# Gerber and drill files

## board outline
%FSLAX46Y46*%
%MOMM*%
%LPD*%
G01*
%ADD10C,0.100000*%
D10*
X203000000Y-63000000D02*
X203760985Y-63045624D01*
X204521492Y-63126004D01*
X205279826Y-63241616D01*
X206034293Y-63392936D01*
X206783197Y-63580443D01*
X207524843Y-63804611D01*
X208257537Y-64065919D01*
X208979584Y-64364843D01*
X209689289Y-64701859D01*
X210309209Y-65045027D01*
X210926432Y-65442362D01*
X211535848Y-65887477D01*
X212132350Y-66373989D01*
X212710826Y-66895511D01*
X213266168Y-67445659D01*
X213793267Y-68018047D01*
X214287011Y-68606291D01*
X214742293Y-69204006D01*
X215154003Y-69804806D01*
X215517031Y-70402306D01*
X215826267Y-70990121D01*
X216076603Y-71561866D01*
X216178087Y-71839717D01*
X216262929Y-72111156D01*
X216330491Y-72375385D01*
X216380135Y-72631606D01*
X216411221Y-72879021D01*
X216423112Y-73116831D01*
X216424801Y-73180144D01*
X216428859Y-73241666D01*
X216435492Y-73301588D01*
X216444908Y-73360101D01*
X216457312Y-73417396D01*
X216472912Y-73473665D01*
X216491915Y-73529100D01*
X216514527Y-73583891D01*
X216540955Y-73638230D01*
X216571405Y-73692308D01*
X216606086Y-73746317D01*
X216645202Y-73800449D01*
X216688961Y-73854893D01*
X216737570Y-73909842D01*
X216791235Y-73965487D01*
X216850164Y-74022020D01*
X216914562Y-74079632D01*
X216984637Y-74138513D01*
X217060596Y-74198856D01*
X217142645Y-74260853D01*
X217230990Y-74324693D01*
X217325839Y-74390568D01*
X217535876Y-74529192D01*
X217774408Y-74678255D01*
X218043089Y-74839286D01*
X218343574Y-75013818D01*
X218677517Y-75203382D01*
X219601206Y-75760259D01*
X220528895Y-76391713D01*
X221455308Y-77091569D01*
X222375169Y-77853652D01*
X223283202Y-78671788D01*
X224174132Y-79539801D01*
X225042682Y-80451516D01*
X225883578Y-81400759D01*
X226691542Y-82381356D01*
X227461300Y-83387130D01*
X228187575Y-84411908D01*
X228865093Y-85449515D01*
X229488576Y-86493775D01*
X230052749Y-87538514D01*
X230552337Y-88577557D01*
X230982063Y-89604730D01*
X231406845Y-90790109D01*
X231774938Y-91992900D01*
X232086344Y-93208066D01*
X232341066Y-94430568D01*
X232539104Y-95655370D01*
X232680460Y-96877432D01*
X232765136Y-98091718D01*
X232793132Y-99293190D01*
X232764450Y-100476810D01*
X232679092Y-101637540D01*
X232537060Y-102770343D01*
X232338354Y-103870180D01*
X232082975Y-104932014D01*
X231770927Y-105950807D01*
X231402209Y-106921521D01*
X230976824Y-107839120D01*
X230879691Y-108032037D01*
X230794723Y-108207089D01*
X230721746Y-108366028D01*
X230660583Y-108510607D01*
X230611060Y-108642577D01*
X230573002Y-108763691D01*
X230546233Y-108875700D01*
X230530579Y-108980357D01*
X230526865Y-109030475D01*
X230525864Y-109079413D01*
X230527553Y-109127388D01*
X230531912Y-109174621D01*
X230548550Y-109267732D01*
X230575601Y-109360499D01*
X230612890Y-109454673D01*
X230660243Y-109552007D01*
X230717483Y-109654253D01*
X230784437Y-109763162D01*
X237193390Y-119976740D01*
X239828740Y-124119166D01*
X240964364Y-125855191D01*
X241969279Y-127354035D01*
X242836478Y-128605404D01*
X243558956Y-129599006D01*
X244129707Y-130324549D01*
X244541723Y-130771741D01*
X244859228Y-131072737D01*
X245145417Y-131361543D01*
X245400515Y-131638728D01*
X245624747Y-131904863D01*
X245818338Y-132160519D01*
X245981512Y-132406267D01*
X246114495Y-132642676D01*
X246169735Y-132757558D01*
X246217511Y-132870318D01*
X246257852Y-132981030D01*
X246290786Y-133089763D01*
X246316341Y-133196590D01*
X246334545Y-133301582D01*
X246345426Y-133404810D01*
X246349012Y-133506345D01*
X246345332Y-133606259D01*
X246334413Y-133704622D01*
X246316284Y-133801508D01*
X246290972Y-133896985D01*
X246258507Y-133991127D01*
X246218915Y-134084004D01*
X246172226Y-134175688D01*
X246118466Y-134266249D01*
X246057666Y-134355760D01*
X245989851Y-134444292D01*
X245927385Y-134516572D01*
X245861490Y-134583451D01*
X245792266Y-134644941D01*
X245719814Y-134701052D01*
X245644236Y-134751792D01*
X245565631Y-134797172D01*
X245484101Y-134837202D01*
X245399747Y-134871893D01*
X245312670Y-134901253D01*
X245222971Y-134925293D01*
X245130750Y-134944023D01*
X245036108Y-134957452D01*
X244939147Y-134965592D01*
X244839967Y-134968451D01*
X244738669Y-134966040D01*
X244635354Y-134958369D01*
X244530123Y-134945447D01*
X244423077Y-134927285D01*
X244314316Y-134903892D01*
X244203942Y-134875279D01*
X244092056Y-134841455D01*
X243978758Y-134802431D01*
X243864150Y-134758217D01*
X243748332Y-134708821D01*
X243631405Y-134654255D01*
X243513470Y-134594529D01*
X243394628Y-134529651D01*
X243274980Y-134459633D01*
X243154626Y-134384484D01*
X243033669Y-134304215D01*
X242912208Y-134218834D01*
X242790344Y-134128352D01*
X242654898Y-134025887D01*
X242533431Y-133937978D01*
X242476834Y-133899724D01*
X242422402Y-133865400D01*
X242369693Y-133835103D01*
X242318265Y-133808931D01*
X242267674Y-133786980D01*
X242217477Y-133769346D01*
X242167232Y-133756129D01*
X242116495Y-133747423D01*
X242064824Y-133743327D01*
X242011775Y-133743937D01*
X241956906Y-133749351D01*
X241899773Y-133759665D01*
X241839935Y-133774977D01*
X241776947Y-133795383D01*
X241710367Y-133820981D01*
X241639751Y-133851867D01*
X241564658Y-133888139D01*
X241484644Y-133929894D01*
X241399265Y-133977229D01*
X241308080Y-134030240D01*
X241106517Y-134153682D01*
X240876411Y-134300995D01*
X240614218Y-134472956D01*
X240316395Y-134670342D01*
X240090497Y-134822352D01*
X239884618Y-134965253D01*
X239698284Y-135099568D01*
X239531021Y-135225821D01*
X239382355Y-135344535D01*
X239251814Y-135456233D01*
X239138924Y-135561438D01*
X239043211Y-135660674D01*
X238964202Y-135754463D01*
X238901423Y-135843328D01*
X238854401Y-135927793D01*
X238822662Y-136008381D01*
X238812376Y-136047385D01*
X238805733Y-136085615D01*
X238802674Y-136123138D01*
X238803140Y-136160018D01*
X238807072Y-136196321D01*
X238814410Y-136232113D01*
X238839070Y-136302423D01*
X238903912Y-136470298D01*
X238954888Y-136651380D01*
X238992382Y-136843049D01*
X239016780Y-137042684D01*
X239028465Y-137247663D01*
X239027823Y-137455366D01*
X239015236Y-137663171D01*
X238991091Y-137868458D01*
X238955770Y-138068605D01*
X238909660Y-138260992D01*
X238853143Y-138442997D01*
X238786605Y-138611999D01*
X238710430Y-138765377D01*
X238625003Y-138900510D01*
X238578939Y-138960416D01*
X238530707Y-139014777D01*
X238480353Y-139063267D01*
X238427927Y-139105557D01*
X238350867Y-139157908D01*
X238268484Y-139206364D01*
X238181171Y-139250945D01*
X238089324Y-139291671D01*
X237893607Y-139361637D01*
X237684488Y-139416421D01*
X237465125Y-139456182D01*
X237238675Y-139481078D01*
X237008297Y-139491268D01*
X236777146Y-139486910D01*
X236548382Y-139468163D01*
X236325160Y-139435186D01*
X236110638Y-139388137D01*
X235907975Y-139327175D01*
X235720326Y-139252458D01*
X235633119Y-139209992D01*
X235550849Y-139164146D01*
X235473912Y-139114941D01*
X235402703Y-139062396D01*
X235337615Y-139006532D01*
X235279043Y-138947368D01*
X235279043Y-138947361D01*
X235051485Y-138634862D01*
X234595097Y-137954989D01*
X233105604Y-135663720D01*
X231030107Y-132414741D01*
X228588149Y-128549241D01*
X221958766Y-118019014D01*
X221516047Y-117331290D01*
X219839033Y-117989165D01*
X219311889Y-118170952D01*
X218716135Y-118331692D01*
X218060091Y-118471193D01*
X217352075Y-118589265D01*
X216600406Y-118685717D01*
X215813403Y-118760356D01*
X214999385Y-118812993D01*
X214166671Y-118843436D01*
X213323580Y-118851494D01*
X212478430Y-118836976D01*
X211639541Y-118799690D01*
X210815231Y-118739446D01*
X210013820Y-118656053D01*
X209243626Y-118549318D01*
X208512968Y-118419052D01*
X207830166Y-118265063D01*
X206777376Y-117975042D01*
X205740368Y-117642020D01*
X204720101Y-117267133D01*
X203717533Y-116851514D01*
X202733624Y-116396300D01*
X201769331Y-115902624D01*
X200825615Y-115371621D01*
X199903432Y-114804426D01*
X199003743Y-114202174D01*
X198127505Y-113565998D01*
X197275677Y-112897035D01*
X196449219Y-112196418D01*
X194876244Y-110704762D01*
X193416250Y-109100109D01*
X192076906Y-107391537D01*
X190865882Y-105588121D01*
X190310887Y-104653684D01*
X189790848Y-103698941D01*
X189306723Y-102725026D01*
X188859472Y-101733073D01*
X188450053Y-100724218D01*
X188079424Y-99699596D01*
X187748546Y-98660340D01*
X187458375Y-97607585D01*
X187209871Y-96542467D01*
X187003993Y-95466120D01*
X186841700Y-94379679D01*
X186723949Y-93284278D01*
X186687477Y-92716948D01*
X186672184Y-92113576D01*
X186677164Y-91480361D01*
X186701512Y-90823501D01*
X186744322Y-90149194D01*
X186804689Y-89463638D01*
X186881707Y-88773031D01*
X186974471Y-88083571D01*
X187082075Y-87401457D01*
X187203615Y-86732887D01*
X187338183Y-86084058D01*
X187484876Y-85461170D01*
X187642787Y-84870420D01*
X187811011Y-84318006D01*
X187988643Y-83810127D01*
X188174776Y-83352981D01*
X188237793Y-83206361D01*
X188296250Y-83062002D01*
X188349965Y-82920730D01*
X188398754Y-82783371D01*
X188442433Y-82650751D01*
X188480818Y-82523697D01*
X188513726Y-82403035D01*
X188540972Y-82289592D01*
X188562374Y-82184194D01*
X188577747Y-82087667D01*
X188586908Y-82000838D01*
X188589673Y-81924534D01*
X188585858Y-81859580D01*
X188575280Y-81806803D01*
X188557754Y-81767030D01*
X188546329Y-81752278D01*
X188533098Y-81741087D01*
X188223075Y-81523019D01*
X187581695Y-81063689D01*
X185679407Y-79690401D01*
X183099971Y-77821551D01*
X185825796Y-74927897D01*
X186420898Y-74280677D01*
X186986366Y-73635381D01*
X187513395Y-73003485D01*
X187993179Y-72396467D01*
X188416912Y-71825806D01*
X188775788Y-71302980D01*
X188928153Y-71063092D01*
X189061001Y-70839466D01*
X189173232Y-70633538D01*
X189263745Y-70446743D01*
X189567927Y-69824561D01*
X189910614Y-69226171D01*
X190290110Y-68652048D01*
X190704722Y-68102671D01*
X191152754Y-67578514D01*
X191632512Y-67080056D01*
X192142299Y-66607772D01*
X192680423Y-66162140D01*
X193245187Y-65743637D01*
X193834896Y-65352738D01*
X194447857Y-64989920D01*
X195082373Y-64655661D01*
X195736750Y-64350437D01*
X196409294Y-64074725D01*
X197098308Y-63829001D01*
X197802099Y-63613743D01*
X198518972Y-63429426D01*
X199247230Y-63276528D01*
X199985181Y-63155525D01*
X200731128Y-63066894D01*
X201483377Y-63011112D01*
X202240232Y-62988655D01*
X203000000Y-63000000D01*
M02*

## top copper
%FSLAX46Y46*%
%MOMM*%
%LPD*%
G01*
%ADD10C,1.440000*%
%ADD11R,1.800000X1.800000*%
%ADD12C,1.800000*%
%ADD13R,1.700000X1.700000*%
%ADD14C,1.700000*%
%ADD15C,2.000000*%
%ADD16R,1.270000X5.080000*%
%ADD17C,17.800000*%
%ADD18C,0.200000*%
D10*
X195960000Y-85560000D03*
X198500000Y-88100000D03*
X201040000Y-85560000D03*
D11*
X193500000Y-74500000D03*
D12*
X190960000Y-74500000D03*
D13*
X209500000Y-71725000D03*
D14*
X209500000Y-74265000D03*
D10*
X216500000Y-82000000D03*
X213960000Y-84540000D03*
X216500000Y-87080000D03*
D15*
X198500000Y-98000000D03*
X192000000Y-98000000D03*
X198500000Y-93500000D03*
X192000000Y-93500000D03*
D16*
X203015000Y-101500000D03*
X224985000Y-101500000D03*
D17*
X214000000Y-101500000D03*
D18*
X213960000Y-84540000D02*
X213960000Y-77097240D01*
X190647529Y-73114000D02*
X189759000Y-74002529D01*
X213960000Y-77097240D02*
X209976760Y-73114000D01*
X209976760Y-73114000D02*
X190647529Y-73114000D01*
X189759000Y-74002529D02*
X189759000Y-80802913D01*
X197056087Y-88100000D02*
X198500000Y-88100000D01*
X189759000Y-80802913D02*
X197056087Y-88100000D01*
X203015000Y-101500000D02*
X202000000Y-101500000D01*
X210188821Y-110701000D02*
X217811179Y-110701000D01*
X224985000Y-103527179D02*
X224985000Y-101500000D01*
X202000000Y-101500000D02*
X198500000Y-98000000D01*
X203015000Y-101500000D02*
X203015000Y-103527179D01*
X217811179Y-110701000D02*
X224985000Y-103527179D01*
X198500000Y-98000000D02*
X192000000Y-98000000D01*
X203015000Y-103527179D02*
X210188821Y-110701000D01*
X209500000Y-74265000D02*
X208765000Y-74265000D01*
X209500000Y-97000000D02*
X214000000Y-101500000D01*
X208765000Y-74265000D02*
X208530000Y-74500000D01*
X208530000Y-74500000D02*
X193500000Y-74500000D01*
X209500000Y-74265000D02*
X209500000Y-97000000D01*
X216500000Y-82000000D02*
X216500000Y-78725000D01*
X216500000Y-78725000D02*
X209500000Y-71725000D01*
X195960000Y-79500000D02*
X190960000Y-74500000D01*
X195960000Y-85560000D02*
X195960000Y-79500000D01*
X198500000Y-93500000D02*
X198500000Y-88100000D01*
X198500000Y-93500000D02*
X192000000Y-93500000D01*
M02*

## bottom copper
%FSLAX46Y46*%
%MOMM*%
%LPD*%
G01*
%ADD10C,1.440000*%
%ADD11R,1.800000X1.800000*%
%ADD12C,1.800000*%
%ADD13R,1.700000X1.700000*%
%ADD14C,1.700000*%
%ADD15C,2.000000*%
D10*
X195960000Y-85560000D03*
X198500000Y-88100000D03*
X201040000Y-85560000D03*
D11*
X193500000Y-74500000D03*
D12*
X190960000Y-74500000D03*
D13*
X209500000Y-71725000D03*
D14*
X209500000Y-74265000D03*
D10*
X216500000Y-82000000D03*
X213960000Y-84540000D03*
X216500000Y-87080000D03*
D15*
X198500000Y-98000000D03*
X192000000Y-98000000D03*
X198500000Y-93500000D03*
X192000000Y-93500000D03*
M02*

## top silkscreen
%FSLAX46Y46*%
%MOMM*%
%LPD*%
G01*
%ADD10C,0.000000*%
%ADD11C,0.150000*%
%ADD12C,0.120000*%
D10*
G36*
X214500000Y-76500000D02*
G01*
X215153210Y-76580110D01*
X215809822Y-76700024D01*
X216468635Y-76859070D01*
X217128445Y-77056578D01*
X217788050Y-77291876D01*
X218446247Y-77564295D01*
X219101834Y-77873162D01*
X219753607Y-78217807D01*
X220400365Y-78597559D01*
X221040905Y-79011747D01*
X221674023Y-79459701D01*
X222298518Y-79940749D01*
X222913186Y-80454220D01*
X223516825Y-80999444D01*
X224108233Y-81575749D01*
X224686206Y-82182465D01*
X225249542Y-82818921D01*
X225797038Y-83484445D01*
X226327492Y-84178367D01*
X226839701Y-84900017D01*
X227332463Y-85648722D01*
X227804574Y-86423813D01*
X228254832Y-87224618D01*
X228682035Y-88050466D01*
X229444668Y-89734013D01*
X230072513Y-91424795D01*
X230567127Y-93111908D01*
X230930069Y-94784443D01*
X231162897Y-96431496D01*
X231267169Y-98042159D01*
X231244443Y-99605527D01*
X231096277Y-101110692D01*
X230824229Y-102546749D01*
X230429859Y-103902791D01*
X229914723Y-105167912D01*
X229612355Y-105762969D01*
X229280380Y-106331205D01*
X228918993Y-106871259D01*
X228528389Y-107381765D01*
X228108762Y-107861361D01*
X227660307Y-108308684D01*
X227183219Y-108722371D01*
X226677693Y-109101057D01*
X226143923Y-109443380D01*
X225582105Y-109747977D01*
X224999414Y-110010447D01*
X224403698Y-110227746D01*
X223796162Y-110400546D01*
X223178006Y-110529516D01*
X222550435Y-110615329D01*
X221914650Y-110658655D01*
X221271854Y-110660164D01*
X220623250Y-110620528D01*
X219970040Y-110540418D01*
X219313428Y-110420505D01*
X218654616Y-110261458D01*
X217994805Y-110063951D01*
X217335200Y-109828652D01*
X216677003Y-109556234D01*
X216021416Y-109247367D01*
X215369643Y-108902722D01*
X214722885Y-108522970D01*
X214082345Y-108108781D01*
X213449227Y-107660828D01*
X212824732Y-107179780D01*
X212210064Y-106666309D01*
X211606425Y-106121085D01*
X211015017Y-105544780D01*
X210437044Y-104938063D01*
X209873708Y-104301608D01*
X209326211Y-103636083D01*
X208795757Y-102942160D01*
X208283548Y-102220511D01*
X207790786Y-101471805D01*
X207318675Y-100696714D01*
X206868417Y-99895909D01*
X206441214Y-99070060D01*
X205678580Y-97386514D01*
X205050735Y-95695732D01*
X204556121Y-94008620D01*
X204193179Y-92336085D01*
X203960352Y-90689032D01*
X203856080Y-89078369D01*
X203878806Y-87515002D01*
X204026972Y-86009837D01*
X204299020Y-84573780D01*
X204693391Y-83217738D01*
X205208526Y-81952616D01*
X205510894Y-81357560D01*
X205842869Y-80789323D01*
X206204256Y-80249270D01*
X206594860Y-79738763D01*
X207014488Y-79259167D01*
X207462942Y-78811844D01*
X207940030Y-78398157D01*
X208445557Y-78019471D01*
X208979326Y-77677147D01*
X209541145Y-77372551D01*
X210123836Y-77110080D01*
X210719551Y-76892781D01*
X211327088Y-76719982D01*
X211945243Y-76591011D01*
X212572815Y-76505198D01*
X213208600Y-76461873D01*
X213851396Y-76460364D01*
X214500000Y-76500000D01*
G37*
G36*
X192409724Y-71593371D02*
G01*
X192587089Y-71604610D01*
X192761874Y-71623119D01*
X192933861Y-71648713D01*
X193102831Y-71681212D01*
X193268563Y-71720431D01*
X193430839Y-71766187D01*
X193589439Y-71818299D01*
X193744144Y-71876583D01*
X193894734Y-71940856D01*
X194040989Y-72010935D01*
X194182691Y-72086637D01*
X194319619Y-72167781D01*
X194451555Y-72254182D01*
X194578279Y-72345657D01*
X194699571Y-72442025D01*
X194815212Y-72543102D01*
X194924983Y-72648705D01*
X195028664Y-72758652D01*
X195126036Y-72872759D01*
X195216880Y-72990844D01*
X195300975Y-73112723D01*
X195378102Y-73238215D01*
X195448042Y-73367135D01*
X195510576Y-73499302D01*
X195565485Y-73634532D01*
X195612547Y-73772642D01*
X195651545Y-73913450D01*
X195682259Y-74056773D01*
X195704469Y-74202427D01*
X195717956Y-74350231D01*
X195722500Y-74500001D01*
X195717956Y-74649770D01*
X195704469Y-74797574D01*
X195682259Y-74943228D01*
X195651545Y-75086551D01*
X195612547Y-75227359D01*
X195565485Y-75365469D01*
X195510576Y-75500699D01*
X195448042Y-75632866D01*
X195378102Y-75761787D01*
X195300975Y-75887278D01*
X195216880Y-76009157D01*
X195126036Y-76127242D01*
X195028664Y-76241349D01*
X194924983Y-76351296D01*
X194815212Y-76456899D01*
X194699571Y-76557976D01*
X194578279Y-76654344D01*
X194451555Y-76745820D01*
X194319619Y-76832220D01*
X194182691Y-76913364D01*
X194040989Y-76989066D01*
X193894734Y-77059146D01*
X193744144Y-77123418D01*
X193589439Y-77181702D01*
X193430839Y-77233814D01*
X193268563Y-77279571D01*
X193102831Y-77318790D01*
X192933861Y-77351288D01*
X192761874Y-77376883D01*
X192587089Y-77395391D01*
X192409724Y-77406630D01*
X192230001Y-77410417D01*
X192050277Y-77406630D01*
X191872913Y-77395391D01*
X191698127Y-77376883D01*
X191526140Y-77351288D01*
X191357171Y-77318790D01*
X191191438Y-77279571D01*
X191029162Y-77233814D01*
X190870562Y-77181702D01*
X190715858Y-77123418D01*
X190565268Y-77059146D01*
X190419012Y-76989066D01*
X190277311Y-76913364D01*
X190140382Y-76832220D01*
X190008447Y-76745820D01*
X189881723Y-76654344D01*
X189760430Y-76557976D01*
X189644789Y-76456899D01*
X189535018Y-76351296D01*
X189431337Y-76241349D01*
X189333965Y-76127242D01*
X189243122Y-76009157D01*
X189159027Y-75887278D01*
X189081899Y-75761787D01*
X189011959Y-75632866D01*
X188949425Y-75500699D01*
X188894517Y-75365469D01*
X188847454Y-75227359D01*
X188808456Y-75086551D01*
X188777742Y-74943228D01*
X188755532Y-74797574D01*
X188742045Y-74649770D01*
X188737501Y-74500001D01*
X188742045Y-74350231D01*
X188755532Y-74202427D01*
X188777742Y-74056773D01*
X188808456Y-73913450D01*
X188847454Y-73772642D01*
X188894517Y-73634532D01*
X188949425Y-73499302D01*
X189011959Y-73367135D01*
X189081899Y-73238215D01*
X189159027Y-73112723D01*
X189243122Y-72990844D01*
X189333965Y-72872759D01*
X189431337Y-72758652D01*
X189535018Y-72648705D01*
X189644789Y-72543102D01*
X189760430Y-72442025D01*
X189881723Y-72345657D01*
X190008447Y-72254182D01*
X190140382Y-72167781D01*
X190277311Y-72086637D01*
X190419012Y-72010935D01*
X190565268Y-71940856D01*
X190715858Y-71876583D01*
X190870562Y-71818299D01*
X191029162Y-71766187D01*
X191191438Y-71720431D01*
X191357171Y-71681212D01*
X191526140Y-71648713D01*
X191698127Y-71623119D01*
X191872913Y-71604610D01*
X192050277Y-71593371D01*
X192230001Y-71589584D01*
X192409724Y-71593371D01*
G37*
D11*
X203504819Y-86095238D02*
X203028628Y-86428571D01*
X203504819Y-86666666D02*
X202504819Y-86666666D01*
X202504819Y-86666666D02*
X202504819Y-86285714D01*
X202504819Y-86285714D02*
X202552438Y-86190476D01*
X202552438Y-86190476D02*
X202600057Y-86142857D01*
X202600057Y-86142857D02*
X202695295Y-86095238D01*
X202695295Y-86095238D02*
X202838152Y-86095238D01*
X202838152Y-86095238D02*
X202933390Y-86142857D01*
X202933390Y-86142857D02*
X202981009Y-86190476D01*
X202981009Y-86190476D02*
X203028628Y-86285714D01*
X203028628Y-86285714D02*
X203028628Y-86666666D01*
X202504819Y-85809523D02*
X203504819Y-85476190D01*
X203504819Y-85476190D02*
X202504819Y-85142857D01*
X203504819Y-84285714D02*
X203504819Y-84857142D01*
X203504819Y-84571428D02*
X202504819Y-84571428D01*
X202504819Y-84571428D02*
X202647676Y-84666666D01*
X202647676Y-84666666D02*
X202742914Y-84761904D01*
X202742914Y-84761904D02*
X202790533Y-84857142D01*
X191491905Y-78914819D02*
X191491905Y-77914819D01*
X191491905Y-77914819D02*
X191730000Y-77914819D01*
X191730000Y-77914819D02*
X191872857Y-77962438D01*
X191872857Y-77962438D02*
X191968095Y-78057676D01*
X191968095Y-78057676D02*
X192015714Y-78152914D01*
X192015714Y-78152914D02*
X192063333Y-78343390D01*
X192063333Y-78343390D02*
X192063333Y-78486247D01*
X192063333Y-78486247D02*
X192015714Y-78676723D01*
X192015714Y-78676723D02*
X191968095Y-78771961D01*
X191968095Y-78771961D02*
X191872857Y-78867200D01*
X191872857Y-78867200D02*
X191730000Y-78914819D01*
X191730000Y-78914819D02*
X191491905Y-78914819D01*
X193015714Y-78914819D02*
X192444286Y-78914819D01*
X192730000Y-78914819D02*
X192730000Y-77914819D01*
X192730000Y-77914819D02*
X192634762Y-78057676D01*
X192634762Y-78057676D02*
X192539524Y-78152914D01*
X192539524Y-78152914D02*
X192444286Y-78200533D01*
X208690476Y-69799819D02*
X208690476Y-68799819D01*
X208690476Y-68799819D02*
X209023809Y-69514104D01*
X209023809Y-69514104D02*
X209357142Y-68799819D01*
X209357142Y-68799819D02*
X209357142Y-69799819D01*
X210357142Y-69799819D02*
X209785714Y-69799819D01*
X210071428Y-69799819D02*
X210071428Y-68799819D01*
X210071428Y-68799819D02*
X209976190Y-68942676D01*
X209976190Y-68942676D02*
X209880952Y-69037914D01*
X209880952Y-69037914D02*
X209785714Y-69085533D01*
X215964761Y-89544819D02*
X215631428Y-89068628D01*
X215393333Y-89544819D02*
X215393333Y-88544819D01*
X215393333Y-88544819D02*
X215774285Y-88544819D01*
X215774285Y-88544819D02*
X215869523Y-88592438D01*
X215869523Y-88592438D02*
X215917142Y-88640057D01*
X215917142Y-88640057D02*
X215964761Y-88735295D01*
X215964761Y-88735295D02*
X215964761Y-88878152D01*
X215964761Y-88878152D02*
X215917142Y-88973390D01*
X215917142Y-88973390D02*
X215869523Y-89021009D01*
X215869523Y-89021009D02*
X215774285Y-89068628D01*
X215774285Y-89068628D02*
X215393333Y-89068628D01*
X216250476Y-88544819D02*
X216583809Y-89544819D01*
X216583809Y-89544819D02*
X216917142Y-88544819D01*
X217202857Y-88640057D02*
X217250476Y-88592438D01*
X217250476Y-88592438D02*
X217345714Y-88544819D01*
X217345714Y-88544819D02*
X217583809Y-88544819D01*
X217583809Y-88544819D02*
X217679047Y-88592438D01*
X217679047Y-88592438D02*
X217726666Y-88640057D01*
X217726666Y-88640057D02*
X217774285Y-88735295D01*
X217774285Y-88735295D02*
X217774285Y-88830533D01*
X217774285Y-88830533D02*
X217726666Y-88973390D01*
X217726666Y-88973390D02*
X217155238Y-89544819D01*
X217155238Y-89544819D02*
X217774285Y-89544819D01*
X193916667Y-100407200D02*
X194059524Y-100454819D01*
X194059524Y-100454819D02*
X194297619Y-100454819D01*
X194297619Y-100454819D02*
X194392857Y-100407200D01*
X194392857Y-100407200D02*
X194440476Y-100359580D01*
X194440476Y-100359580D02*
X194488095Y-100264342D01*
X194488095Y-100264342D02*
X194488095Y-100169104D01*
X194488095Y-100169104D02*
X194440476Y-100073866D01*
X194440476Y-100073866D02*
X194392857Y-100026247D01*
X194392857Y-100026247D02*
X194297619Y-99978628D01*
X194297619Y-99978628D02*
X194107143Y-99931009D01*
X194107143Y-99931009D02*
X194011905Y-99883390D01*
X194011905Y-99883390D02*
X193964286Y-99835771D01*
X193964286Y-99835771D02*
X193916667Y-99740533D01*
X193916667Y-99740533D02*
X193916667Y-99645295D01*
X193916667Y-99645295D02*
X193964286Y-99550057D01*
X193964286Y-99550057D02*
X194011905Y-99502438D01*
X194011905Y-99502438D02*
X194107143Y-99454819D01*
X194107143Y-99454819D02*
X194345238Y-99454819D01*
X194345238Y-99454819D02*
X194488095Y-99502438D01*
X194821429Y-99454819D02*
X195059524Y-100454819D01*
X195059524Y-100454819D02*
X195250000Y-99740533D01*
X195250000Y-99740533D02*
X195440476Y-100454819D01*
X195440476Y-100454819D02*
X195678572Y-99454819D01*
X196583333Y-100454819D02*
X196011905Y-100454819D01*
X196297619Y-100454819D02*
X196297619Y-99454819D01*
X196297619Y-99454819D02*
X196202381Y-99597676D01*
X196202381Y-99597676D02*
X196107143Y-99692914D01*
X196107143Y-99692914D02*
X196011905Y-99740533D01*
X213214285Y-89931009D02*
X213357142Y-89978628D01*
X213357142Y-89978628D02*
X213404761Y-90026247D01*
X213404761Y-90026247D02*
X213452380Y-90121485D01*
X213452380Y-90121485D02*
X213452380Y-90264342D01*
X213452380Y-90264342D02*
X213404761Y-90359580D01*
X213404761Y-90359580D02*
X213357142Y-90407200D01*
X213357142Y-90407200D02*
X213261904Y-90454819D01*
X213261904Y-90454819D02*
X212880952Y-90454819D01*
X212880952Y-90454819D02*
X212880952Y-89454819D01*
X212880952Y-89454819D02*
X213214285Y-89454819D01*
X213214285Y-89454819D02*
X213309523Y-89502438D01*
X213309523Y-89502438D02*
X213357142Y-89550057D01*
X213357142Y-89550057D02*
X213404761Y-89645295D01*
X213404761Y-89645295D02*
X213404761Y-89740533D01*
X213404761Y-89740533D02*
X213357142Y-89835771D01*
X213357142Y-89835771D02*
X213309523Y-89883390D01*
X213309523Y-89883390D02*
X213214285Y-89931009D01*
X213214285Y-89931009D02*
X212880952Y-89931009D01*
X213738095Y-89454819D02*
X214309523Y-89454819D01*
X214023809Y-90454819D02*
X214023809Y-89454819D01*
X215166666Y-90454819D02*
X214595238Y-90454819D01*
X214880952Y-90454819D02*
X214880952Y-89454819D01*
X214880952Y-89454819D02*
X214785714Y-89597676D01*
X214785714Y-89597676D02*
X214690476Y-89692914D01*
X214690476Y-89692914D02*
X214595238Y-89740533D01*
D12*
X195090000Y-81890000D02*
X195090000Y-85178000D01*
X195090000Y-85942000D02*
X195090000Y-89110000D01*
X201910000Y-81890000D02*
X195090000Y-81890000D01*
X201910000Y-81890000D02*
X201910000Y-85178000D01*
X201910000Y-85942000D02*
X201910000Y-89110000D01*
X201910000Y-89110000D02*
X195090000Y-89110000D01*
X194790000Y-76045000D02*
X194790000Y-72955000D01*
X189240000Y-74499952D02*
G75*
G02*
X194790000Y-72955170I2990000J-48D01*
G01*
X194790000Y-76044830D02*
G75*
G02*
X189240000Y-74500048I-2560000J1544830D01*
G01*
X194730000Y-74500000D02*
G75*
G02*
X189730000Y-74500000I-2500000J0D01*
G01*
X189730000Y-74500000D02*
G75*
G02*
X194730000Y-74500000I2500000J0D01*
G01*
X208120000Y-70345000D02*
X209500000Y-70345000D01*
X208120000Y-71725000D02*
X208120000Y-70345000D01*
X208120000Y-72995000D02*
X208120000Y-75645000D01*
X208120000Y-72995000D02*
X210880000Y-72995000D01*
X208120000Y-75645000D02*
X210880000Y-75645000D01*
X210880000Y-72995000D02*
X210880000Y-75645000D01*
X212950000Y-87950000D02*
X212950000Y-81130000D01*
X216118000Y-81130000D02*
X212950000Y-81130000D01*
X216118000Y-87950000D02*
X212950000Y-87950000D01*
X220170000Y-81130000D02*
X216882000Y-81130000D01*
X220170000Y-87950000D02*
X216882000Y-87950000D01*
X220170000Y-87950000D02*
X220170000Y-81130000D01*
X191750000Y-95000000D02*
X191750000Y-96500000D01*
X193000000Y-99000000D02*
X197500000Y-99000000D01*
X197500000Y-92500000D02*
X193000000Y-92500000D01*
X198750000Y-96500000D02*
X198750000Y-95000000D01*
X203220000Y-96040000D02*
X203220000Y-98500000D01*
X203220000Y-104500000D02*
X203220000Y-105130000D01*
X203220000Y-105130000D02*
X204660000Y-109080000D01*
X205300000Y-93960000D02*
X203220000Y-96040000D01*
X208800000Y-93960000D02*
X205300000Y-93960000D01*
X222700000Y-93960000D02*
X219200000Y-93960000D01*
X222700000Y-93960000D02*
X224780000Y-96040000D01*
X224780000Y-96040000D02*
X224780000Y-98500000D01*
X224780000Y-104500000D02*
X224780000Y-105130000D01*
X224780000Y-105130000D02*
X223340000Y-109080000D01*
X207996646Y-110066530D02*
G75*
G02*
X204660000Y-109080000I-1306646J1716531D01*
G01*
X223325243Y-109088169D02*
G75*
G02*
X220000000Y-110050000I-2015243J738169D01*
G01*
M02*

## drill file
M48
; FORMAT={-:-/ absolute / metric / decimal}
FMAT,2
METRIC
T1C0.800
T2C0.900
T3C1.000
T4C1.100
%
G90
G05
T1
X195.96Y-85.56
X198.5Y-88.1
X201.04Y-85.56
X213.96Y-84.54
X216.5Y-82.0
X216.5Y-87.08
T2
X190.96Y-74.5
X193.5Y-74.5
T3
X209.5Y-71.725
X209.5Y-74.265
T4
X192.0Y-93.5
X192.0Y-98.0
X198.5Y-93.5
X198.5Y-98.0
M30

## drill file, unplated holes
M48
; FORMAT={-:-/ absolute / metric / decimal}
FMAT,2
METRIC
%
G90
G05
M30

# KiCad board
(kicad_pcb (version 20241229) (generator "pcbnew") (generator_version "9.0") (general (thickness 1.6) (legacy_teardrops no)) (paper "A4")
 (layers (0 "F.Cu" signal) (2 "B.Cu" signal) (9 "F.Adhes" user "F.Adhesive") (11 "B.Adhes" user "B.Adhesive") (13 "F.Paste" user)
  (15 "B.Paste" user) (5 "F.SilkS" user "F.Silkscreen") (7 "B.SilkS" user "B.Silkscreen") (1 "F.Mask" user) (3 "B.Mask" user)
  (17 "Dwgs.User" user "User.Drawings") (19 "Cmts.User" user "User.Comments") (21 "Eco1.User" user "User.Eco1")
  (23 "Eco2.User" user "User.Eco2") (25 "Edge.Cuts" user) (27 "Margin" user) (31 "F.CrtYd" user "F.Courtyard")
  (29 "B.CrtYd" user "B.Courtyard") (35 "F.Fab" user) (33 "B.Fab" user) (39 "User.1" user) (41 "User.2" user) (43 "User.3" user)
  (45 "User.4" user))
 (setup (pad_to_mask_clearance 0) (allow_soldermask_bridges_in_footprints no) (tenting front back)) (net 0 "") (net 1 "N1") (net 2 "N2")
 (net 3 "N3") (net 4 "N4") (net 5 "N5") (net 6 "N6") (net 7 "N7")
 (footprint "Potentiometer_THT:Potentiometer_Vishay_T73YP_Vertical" (layer "F.Cu") (at 195.96 85.56 -90)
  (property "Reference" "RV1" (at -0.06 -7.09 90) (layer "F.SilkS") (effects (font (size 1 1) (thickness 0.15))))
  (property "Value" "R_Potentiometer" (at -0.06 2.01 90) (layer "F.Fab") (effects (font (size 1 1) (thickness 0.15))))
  (fp_line (start -3.67 0.87) (end -0.382 0.87) (stroke (width 0.12) (type solid)) (layer "F.SilkS"))
  (fp_line (start 0.382 0.87) (end 3.55 0.87) (stroke (width 0.12) (type solid)) (layer "F.SilkS"))
  (fp_line (start -3.67 -5.95) (end -3.67 0.87) (stroke (width 0.12) (type solid)) (layer "F.SilkS"))
  (fp_line (start -3.67 -5.95) (end -0.382 -5.95) (stroke (width 0.12) (type solid)) (layer "F.SilkS"))
  (fp_line (start 0.382 -5.95) (end 3.55 -5.95) (stroke (width 0.12) (type solid)) (layer "F.SilkS"))
  (fp_line (start 3.55 -5.95) (end 3.55 0.87) (stroke (width 0.12) (type solid)) (layer "F.SilkS"))
  (pad "1" thru_hole circle (at 0 0 270) (size 1.44 1.44) (drill 0.8) (layers "*.Cu" "*.Mask") (remove_unused_layers no) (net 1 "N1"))
  (pad "2" thru_hole circle (at 2.54 -2.54 270) (size 1.44 1.44) (drill 0.8) (layers "*.Cu" "*.Mask") (remove_unused_layers no) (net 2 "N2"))
  (pad "3" thru_hole circle (at 0 -5.08 270) (size 1.44 1.44) (drill 0.8) (layers "*.Cu" "*.Mask") (remove_unused_layers no) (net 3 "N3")))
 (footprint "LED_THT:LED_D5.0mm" (layer "F.Cu") (at 193.5 74.5 180)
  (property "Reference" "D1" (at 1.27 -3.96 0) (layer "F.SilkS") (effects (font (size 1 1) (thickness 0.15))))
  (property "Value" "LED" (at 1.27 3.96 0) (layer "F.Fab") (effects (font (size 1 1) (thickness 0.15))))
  (fp_line (start -1.29 -1.545) (end -1.29 1.545) (stroke (width 0.12) (type solid)) (layer "F.SilkS"))
  (fp_arc (start 4.26 0.000048) (mid 2.071756 2.880501) (end -1.29 1.54483) (stroke (width 0.12) (type solid)) (layer "F.SilkS"))
  (fp_arc (start -1.29 -1.54483) (mid 2.071756 -2.880501) (end 4.26 -0.000048) (stroke (width 0.12) (type solid)) (layer "F.SilkS"))
  (fp_circle (center 1.27 0) (end 3.77 0) (stroke (width 0.12) (type solid)) (fill no) (layer "F.SilkS"))
  (pad "1" thru_hole rect (at 0 0 180) (size 1.8 1.8) (drill 0.9) (layers "*.Cu" "*.Mask") (remove_unused_layers no) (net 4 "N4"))
  (pad "2" thru_hole circle (at 2.54 0 180) (size 1.8 1.8) (drill 0.9) (layers "*.Cu" "*.Mask") (remove_unused_layers no) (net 1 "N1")))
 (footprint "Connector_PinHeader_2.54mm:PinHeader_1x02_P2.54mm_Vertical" (layer "F.Cu") (at 209.5 71.725)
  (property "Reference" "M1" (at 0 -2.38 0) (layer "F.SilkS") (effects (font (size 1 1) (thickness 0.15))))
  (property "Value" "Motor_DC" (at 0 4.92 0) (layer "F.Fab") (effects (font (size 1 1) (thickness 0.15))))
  (fp_line (start -1.38 -1.38) (end 0 -1.38) (stroke (width 0.12) (type solid)) (layer "F.SilkS"))
  (fp_line (start -1.38 0) (end -1.38 -1.38) (stroke (width 0.12) (type solid)) (layer "F.SilkS"))
  (fp_line (start -1.38 1.27) (end -1.38 3.92) (stroke (width 0.12) (type solid)) (layer "F.SilkS"))
  (fp_line (start -1.38 1.27) (end 1.38 1.27) (stroke (width 0.12) (type solid)) (layer "F.SilkS"))
  (fp_line (start -1.38 3.92) (end 1.38 3.92) (stroke (width 0.12) (type solid)) (layer "F.SilkS"))
  (fp_line (start 1.38 1.27) (end 1.38 3.92) (stroke (width 0.12) (type solid)) (layer "F.SilkS"))
  (pad "1" thru_hole rect (at 0 0) (size 1.7 1.7) (drill 1) (layers "*.Cu" "*.Mask") (remove_unused_layers no) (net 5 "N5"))
  (pad "2" thru_hole circle (at 0 2.54) (size 1.7 1.7) (drill 1) (layers "*.Cu" "*.Mask") (remove_unused_layers no) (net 4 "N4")))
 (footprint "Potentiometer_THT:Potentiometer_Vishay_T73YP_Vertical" (layer "F.Cu") (at 216.5 82 180)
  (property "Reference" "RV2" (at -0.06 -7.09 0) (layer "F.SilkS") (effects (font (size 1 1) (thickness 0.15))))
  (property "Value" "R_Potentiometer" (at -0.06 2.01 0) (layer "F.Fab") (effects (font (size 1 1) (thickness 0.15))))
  (fp_line (start 3.55 -5.95) (end 3.55 0.87) (stroke (width 0.12) (type solid)) (layer "F.SilkS"))
  (fp_line (start 0.382 0.87) (end 3.55 0.87) (stroke (width 0.12) (type solid)) (layer "F.SilkS"))
  (fp_line (start 0.382 -5.95) (end 3.55 -5.95) (stroke (width 0.12) (type solid)) (layer "F.SilkS"))
  (fp_line (start -3.67 0.87) (end -0.382 0.87) (stroke (width 0.12) (type solid)) (layer "F.SilkS"))
  (fp_line (start -3.67 -5.95) (end -0.382 -5.95) (stroke (width 0.12) (type solid)) (layer "F.SilkS"))
  (fp_line (start -3.67 -5.95) (end -3.67 0.87) (stroke (width 0.12) (type solid)) (layer "F.SilkS"))
  (pad "1" thru_hole circle (at 0 0 180) (size 1.44 1.44) (drill 0.8) (layers "*.Cu" "*.Mask") (remove_unused_layers no) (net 5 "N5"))
  (pad "2" thru_hole circle (at 2.54 -2.54 180) (size 1.44 1.44) (drill 0.8) (layers "*.Cu" "*.Mask") (remove_unused_layers no) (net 2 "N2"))
  (pad "3" thru_hole circle (at 0 -5.08 180) (size 1.44 1.44) (drill 0.8) (layers "*.Cu" "*.Mask") (remove_unused_layers no) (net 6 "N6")))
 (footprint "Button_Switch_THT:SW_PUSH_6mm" (layer "F.Cu") (at 198.5 98 180)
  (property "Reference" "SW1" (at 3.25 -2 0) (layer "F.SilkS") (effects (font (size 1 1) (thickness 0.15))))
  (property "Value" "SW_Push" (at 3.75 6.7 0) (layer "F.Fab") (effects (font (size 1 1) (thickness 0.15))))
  (fp_line (start 6.75 3) (end 6.75 1.5) (stroke (width 0.12) (type solid)) (layer "F.SilkS"))
  (fp_line (start 5.5 -1) (end 1 -1) (stroke (width 0.12) (type solid)) (layer "F.SilkS"))
  (fp_line (start 1 5.5) (end 5.5 5.5) (stroke (width 0.12) (type solid)) (layer "F.SilkS"))
  (fp_line (start -0.25 1.5) (end -0.25 3) (stroke (width 0.12) (type solid)) (layer "F.SilkS"))
  (pad "1" thru_hole circle (at 0 0 270) (size 2 2) (drill 1.1) (layers "*.Cu" "*.Mask") (remove_unused_layers no) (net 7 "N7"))
  (pad "1" thru_hole circle (at 6.5 0 270) (size 2 2) (drill 1.1) (layers "*.Cu" "*.Mask") (remove_unused_layers no) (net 7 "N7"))
  (pad "2" thru_hole circle (at 0 4.5 270) (size 2 2) (drill 1.1) (layers "*.Cu" "*.Mask") (remove_unused_layers no) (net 2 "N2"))
  (pad "2" thru_hole circle (at 6.5 4.5 270) (size 2 2) (drill 1.1) (layers "*.Cu" "*.Mask") (remove_unused_layers no) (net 2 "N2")))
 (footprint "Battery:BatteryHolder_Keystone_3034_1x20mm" (layer "F.Cu") (at 214 101.5)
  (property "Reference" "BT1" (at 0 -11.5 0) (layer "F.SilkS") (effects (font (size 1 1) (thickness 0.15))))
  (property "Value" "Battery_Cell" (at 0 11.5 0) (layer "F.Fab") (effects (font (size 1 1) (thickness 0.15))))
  (fp_line (start -10.78 -5.46) (end -10.78 -3) (stroke (width 0.12) (type solid)) (layer "F.SilkS"))
  (fp_line (start -10.78 3) (end -10.78 3.63) (stroke (width 0.12) (type solid)) (layer "F.SilkS"))
  (fp_line (start -10.78 3.63) (end -9.34 7.58) (stroke (width 0.12) (type solid)) (layer "F.SilkS"))
  (fp_line (start -8.7 -7.54) (end -10.78 -5.46) (stroke (width 0.12) (type solid)) (layer "F.SilkS"))
  (fp_line (start -5.2 -7.54) (end -8.7 -7.54) (stroke (width 0.12) (type solid)) (layer "F.SilkS"))
  (fp_line (start 8.7 -7.54) (end 5.2 -7.54) (stroke (width 0.12) (type solid)) (layer "F.SilkS"))
  (fp_line (start 8.7 -7.54) (end 10.78 -5.46) (stroke (width 0.12) (type solid)) (layer "F.SilkS"))
  (fp_line (start 10.78 -5.46) (end 10.78 -3) (stroke (width 0.12) (type solid)) (layer "F.SilkS"))
  (fp_line (start 10.78 3) (end 10.78 3.63) (stroke (width 0.12) (type solid)) (layer "F.SilkS"))
  (fp_line (start 10.78 3.63) (end 9.34 7.58) (stroke (width 0.12) (type solid)) (layer "F.SilkS"))
  (fp_arc (start -6.003354 8.56653) (mid -7.921654 8.918738) (end -9.34 7.58) (stroke (width 0.12) (type solid)) (layer "F.SilkS"))
  (fp_arc (start 9.325243 7.588169) (mid 7.90634 8.911668) (end 6 8.55) (stroke (width 0.12) (type solid)) (layer "F.SilkS"))
  (pad "1" smd rect (at -10.985 0) (size 1.27 5.08) (layers "F.Cu" "F.Mask" "F.Paste") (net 7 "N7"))
  (pad "1" smd rect (at 10.985 0) (size 1.27 5.08) (layers "F.Cu" "F.Mask" "F.Paste") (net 7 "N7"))
  (pad "2" smd circle (at 0 0) (size 17.8 17.8) (layers "F.Cu" "F.Mask") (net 4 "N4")))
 (gr_poly
  (pts (xy 214.5 76.5) (xy 215.15321 76.58011) (xy 215.809822 76.700024) (xy 216.468635 76.85907) (xy 217.128445 77.056578)
   (xy 217.78805 77.291876) (xy 218.446247 77.564295) (xy 219.101834 77.873162) (xy 219.753607 78.217807) (xy 220.400365 78.597559)
   (xy 221.040905 79.011747) (xy 221.674023 79.459701) (xy 222.298518 79.940749) (xy 222.913186 80.45422) (xy 223.516825 80.999444)
   (xy 224.108233 81.575749) (xy 224.686206 82.182465) (xy 225.249542 82.818921) (xy 225.797038 83.484445) (xy 226.327492 84.178367)
   (xy 226.839701 84.900017) (xy 227.332463 85.648722) (xy 227.804574 86.423813) (xy 228.254832 87.224618) (xy 228.682035 88.050466)
   (xy 229.444668 89.734013) (xy 230.072513 91.424795) (xy 230.567127 93.111908) (xy 230.930069 94.784443) (xy 231.162897 96.431496)
   (xy 231.267169 98.042159) (xy 231.244443 99.605527) (xy 231.096277 101.110692) (xy 230.824229 102.546749) (xy 230.429859 103.902791)
   (xy 229.914723 105.167912) (xy 229.612355 105.762969) (xy 229.28038 106.331205) (xy 228.918993 106.871259) (xy 228.528389 107.381765)
   (xy 228.108762 107.861361) (xy 227.660307 108.308684) (xy 227.183219 108.722371) (xy 226.677693 109.101057) (xy 226.143923 109.44338)
   (xy 225.582105 109.747977) (xy 224.999414 110.010447) (xy 224.403698 110.227746) (xy 223.796162 110.400546) (xy 223.178006 110.529516)
   (xy 222.550435 110.615329) (xy 221.91465 110.658655) (xy 221.271854 110.660164) (xy 220.62325 110.620528) (xy 219.97004 110.540418)
   (xy 219.313428 110.420505) (xy 218.654616 110.261458) (xy 217.994805 110.063951) (xy 217.3352 109.828652) (xy 216.677003 109.556234)
   (xy 216.021416 109.247367) (xy 215.369643 108.902722) (xy 214.722885 108.52297) (xy 214.082345 108.108781) (xy 213.449227 107.660828)
   (xy 212.824732 107.17978) (xy 212.210064 106.666309) (xy 211.606425 106.121085) (xy 211.015017 105.54478) (xy 210.437044 104.938063)
   (xy 209.873708 104.301608) (xy 209.326211 103.636083) (xy 208.795757 102.94216) (xy 208.283548 102.220511) (xy 207.790786 101.471805)
   (xy 207.318675 100.696714) (xy 206.868417 99.895909) (xy 206.441214 99.07006) (xy 205.67858 97.386514) (xy 205.050735 95.695732)
   (xy 204.556121 94.00862) (xy 204.193179 92.336085) (xy 203.960352 90.689032) (xy 203.85608 89.078369) (xy 203.878806 87.515002)
   (xy 204.026972 86.009837) (xy 204.29902 84.57378) (xy 204.693391 83.217738) (xy 205.208526 81.952616) (xy 205.510894 81.35756)
   (xy 205.842869 80.789323) (xy 206.204256 80.24927) (xy 206.59486 79.738763) (xy 207.014488 79.259167) (xy 207.462942 78.811844)
   (xy 207.94003 78.398157) (xy 208.445557 78.019471) (xy 208.979326 77.677147) (xy 209.541145 77.372551) (xy 210.123836 77.11008)
   (xy 210.719551 76.892781) (xy 211.327088 76.719982) (xy 211.945243 76.591011) (xy 212.572815 76.505198) (xy 213.2086 76.461873)
   (xy 213.851396 76.460364))
  (stroke (width 0) (type solid)) (fill yes) (layer "F.SilkS"))
 (gr_poly
  (pts (xy 192.409724 71.593371) (xy 192.587089 71.60461) (xy 192.761874 71.623119) (xy 192.933861 71.648713) (xy 193.102831 71.681212)
   (xy 193.268563 71.720431) (xy 193.430839 71.766187) (xy 193.589439 71.818299) (xy 193.744144 71.876583) (xy 193.894734 71.940856)
   (xy 194.040989 72.010935) (xy 194.182691 72.086637) (xy 194.319619 72.167781) (xy 194.451555 72.254182) (xy 194.578279 72.345657)
   (xy 194.699571 72.442025) (xy 194.815212 72.543102) (xy 194.924983 72.648705) (xy 195.028664 72.758652) (xy 195.126036 72.872759)
   (xy 195.21688 72.990844) (xy 195.300975 73.112723) (xy 195.378102 73.238215) (xy 195.448042 73.367135) (xy 195.510576 73.499302)
   (xy 195.565485 73.634532) (xy 195.612547 73.772642) (xy 195.651545 73.91345) (xy 195.682259 74.056773) (xy 195.704469 74.202427)
   (xy 195.717956 74.350231) (xy 195.7225 74.500001) (xy 195.717956 74.64977) (xy 195.704469 74.797574) (xy 195.682259 74.943228)
   (xy 195.651545 75.086551) (xy 195.612547 75.227359) (xy 195.565485 75.365469) (xy 195.510576 75.500699) (xy 195.448042 75.632866)
   (xy 195.378102 75.761787) (xy 195.300975 75.887278) (xy 195.21688 76.009157) (xy 195.126036 76.127242) (xy 195.028664 76.241349)
   (xy 194.924983 76.351296) (xy 194.815212 76.456899) (xy 194.699571 76.557976) (xy 194.578279 76.654344) (xy 194.451555 76.74582)
   (xy 194.319619 76.83222) (xy 194.182691 76.913364) (xy 194.040989 76.989066) (xy 193.894734 77.059146) (xy 193.744144 77.123418)
   (xy 193.589439 77.181702) (xy 193.430839 77.233814) (xy 193.268563 77.279571) (xy 193.102831 77.31879) (xy 192.933861 77.351288)
   (xy 192.761874 77.376883) (xy 192.587089 77.395391) (xy 192.409724 77.40663) (xy 192.230001 77.410417) (xy 192.050277 77.40663)
   (xy 191.872913 77.395391) (xy 191.698127 77.376883) (xy 191.52614 77.351288) (xy 191.357171 77.31879) (xy 191.191438 77.279571)
   (xy 191.029162 77.233814) (xy 190.870562 77.181702) (xy 190.715858 77.123418) (xy 190.565268 77.059146) (xy 190.419012 76.989066)
   (xy 190.277311 76.913364) (xy 190.140382 76.83222) (xy 190.008447 76.74582) (xy 189.881723 76.654344) (xy 189.76043 76.557976)
   (xy 189.644789 76.456899) (xy 189.535018 76.351296) (xy 189.431337 76.241349) (xy 189.333965 76.127242) (xy 189.243122 76.009157)
   (xy 189.159027 75.887278) (xy 189.081899 75.761787) (xy 189.011959 75.632866) (xy 188.949425 75.500699) (xy 188.894517 75.365469)
   (xy 188.847454 75.227359) (xy 188.808456 75.086551) (xy 188.777742 74.943228) (xy 188.755532 74.797574) (xy 188.742045 74.64977)
   (xy 188.737501 74.500001) (xy 188.742045 74.350231) (xy 188.755532 74.202427) (xy 188.777742 74.056773) (xy 188.808456 73.91345)
   (xy 188.847454 73.772642) (xy 188.894517 73.634532) (xy 188.949425 73.499302) (xy 189.011959 73.367135) (xy 189.081899 73.238215)
   (xy 189.159027 73.112723) (xy 189.243122 72.990844) (xy 189.333965 72.872759) (xy 189.431337 72.758652) (xy 189.535018 72.648705)
   (xy 189.644789 72.543102) (xy 189.76043 72.442025) (xy 189.881723 72.345657) (xy 190.008447 72.254182) (xy 190.140382 72.167781)
   (xy 190.277311 72.086637) (xy 190.419012 72.010935) (xy 190.565268 71.940856) (xy 190.715858 71.876583) (xy 190.870562 71.818299)
   (xy 191.029162 71.766187) (xy 191.191438 71.720431) (xy 191.357171 71.681212) (xy 191.52614 71.648713) (xy 191.698127 71.623119)
   (xy 191.872913 71.60461) (xy 192.050277 71.593371) (xy 192.230001 71.589584))
  (stroke (width 0) (type solid)) (fill yes) (layer "F.SilkS"))
 (gr_poly
  (pts (xy 203 63) (xy 203.760985 63.045624) (xy 204.521492 63.126004) (xy 205.279826 63.241616) (xy 206.034293 63.392936)
   (xy 206.783197 63.580443) (xy 207.524843 63.804611) (xy 208.257537 64.065919) (xy 208.979584 64.364843) (xy 209.689289 64.701859)
   (xy 210.309209 65.045027) (xy 210.926432 65.442362) (xy 211.535848 65.887477) (xy 212.13235 66.373989) (xy 212.710826 66.895511)
   (xy 213.266168 67.445659) (xy 213.793267 68.018047) (xy 214.287011 68.606291) (xy 214.742293 69.204006) (xy 215.154003 69.804806)
   (xy 215.517031 70.402306) (xy 215.826267 70.990121) (xy 216.076603 71.561866) (xy 216.178087 71.839717) (xy 216.262929 72.111156)
   (xy 216.330491 72.375385) (xy 216.380135 72.631606) (xy 216.411221 72.879021) (xy 216.423112 73.116831) (xy 216.424801 73.180144)
   (xy 216.428859 73.241666) (xy 216.435492 73.301588) (xy 216.444908 73.360101) (xy 216.457312 73.417396) (xy 216.472912 73.473665)
   (xy 216.491915 73.5291) (xy 216.514527 73.583891) (xy 216.540955 73.63823) (xy 216.571405 73.692308) (xy 216.606086 73.746317)
   (xy 216.645202 73.800449) (xy 216.688961 73.854893) (xy 216.73757 73.909842) (xy 216.791235 73.965487) (xy 216.850164 74.02202)
   (xy 216.914562 74.079632) (xy 216.984637 74.138513) (xy 217.060596 74.198856) (xy 217.142645 74.260853) (xy 217.23099 74.324693)
   (xy 217.325839 74.390568) (xy 217.535876 74.529192) (xy 217.774408 74.678255) (xy 218.043089 74.839286) (xy 218.343574 75.013818)
   (xy 218.677517 75.203382) (xy 219.601206 75.760259) (xy 220.528895 76.391713) (xy 221.455308 77.091569) (xy 222.375169 77.853652)
   (xy 223.283202 78.671788) (xy 224.174132 79.539801) (xy 225.042682 80.451516) (xy 225.883578 81.400759) (xy 226.691542 82.381356)
   (xy 227.4613 83.38713) (xy 228.187575 84.411908) (xy 228.865093 85.449515) (xy 229.488576 86.493775) (xy 230.052749 87.538514)
   (xy 230.552337 88.577557) (xy 230.982063 89.60473) (xy 231.406845 90.790109) (xy 231.774938 91.9929) (xy 232.086344 93.208066)
   (xy 232.341066 94.430568) (xy 232.539104 95.65537) (xy 232.68046 96.877432) (xy 232.765136 98.091718) (xy 232.793132 99.29319)
   (xy 232.76445 100.47681) (xy 232.679092 101.63754) (xy 232.53706 102.770343) (xy 232.338354 103.87018) (xy 232.082975 104.932014)
   (xy 231.770927 105.950807) (xy 231.402209 106.921521) (xy 230.976824 107.83912) (xy 230.879691 108.032037) (xy 230.794723 108.207089)
   (xy 230.721746 108.366028) (xy 230.660583 108.510607) (xy 230.61106 108.642577) (xy 230.573002 108.763691) (xy 230.546233 108.8757)
   (xy 230.530579 108.980357) (xy 230.526865 109.030475) (xy 230.525864 109.079413) (xy 230.527553 109.127388) (xy 230.531912 109.174621)
   (xy 230.54855 109.267732) (xy 230.575601 109.360499) (xy 230.61289 109.454673) (xy 230.660243 109.552007) (xy 230.717483 109.654253)
   (xy 230.784437 109.763162) (xy 237.19339 119.97674) (xy 239.82874 124.119166) (xy 240.964364 125.855191) (xy 241.969279 127.354035)
   (xy 242.836478 128.605404) (xy 243.558956 129.599006) (xy 244.129707 130.324549) (xy 244.541723 130.771741) (xy 244.859228 131.072737)
   (xy 245.145417 131.361543) (xy 245.400515 131.638728) (xy 245.624747 131.904863) (xy 245.818338 132.160519) (xy 245.981512 132.406267)
   (xy 246.114495 132.642676) (xy 246.169735 132.757558) (xy 246.217511 132.870318) (xy 246.257852 132.98103) (xy 246.290786 133.089763)
   (xy 246.316341 133.19659) (xy 246.334545 133.301582) (xy 246.345426 133.40481) (xy 246.349012 133.506345) (xy 246.345332 133.606259)
   (xy 246.334413 133.704622) (xy 246.316284 133.801508) (xy 246.290972 133.896985) (xy 246.258507 133.991127) (xy 246.218915 134.084004)
   (xy 246.172226 134.175688) (xy 246.118466 134.266249) (xy 246.057666 134.35576) (xy 245.989851 134.444292) (xy 245.927385 134.516572)
   (xy 245.86149 134.583451) (xy 245.792266 134.644941) (xy 245.719814 134.701052) (xy 245.644236 134.751792) (xy 245.565631 134.797172)
   (xy 245.484101 134.837202) (xy 245.399747 134.871893) (xy 245.31267 134.901253) (xy 245.222971 134.925293) (xy 245.13075 134.944023)
   (xy 245.036108 134.957452) (xy 244.939147 134.965592) (xy 244.839967 134.968451) (xy 244.738669 134.96604) (xy 244.635354 134.958369)
   (xy 244.530123 134.945447) (xy 244.423077 134.927285) (xy 244.314316 134.903892) (xy 244.203942 134.875279) (xy 244.092056 134.841455)
   (xy 243.978758 134.802431) (xy 243.86415 134.758217) (xy 243.748332 134.708821) (xy 243.631405 134.654255) (xy 243.51347 134.594529)
   (xy 243.394628 134.529651) (xy 243.27498 134.459633) (xy 243.154626 134.384484) (xy 243.033669 134.304215) (xy 242.912208 134.218834)
   (xy 242.790344 134.128352) (xy 242.654898 134.025887) (xy 242.533431 133.937978) (xy 242.476834 133.899724) (xy 242.422402 133.8654)
   (xy 242.369693 133.835103) (xy 242.318265 133.808931) (xy 242.267674 133.78698) (xy 242.217477 133.769346) (xy 242.167232 133.756129)
   (xy 242.116495 133.747423) (xy 242.064824 133.743327) (xy 242.011775 133.743937) (xy 241.956906 133.749351) (xy 241.899773 133.759665)
   (xy 241.839935 133.774977) (xy 241.776947 133.795383) (xy 241.710367 133.820981) (xy 241.639751 133.851867) (xy 241.564658 133.888139)
   (xy 241.484644 133.929894) (xy 241.399265 133.977229) (xy 241.30808 134.03024) (xy 241.106517 134.153682) (xy 240.876411 134.300995)
   (xy 240.614218 134.472956) (xy 240.316395 134.670342) (xy 240.090497 134.822352) (xy 239.884618 134.965253) (xy 239.698284 135.099568)
   (xy 239.531021 135.225821) (xy 239.382355 135.344535) (xy 239.251814 135.456233) (xy 239.138924 135.561438) (xy 239.043211 135.660674)
   (xy 238.964202 135.754463) (xy 238.901423 135.843328) (xy 238.854401 135.927793) (xy 238.822662 136.008381) (xy 238.812376 136.047385)
   (xy 238.805733 136.085615) (xy 238.802674 136.123138) (xy 238.80314 136.160018) (xy 238.807072 136.196321) (xy 238.81441 136.232113)
   (xy 238.83907 136.302423) (xy 238.903912 136.470298) (xy 238.954888 136.65138) (xy 238.992382 136.843049) (xy 239.01678 137.042684)
   (xy 239.028465 137.247663) (xy 239.027823 137.455366) (xy 239.015236 137.663171) (xy 238.991091 137.868458) (xy 238.95577 138.068605)
   (xy 238.90966 138.260992) (xy 238.853143 138.442997) (xy 238.786605 138.611999) (xy 238.71043 138.765377) (xy 238.625003 138.90051)
   (xy 238.578939 138.960416) (xy 238.530707 139.014777) (xy 238.480353 139.063267) (xy 238.427927 139.105557) (xy 238.350867 139.157908)
   (xy 238.268484 139.206364) (xy 238.181171 139.250945) (xy 238.089324 139.291671) (xy 237.893607 139.361637) (xy 237.684488 139.416421)
   (xy 237.465125 139.456182) (xy 237.238675 139.481078) (xy 237.008297 139.491268) (xy 236.777146 139.48691) (xy 236.548382 139.468163)
   (xy 236.32516 139.435186) (xy 236.110638 139.388137) (xy 235.907975 139.327175) (xy 235.720326 139.252458) (xy 235.633119 139.209992)
   (xy 235.550849 139.164146) (xy 235.473912 139.114941) (xy 235.402703 139.062396) (xy 235.337615 139.006532) (xy 235.279043 138.947368)
   (xy 235.279043 138.947361) (xy 235.051485 138.634862) (xy 234.595097 137.954989) (xy 233.105604 135.66372) (xy 231.030107 132.414741)
   (xy 228.588149 128.549241) (xy 221.958766 118.019014) (xy 221.516047 117.33129) (xy 219.839033 117.989165) (xy 219.311889 118.170952)
   (xy 218.716135 118.331692) (xy 218.060091 118.471193) (xy 217.352075 118.589265) (xy 216.600406 118.685717) (xy 215.813403 118.760356)
   (xy 214.999385 118.812993) (xy 214.166671 118.843436) (xy 213.32358 118.851494) (xy 212.47843 118.836976) (xy 211.639541 118.79969)
   (xy 210.815231 118.739446) (xy 210.01382 118.656053) (xy 209.243626 118.549318) (xy 208.512968 118.419052) (xy 207.830166 118.265063)
   (xy 206.777376 117.975042) (xy 205.740368 117.64202) (xy 204.720101 117.267133) (xy 203.717533 116.851514) (xy 202.733624 116.3963)
   (xy 201.769331 115.902624) (xy 200.825615 115.371621) (xy 199.903432 114.804426) (xy 199.003743 114.202174) (xy 198.127505 113.565998)
   (xy 197.275677 112.897035) (xy 196.449219 112.196418) (xy 194.876244 110.704762) (xy 193.41625 109.100109) (xy 192.076906 107.391537)
   (xy 190.865882 105.588121) (xy 190.310887 104.653684) (xy 189.790848 103.698941) (xy 189.306723 102.725026) (xy 188.859472 101.733073)
   (xy 188.450053 100.724218) (xy 188.079424 99.699596) (xy 187.748546 98.66034) (xy 187.458375 97.607585) (xy 187.209871 96.542467)
   (xy 187.003993 95.46612) (xy 186.8417 94.379679) (xy 186.723949 93.284278) (xy 186.687477 92.716948) (xy 186.672184 92.113576)
   (xy 186.677164 91.480361) (xy 186.701512 90.823501) (xy 186.744322 90.149194) (xy 186.804689 89.463638) (xy 186.881707 88.773031)
   (xy 186.974471 88.083571) (xy 187.082075 87.401457) (xy 187.203615 86.732887) (xy 187.338183 86.084058) (xy 187.484876 85.46117)
   (xy 187.642787 84.87042) (xy 187.811011 84.318006) (xy 187.988643 83.810127) (xy 188.174776 83.352981) (xy 188.237793 83.206361)
   (xy 188.29625 83.062002) (xy 188.349965 82.92073) (xy 188.398754 82.783371) (xy 188.442433 82.650751) (xy 188.480818 82.523697)
   (xy 188.513726 82.403035) (xy 188.540972 82.289592) (xy 188.562374 82.184194) (xy 188.577747 82.087667) (xy 188.586908 82.000838)
   (xy 188.589673 81.924534) (xy 188.585858 81.85958) (xy 188.57528 81.806803) (xy 188.557754 81.76703) (xy 188.546329 81.752278)
   (xy 188.533098 81.741087) (xy 188.223075 81.523019) (xy 187.581695 81.063689) (xy 185.679407 79.690401) (xy 183.099971 77.821551)
   (xy 185.825796 74.927897) (xy 186.420898 74.280677) (xy 186.986366 73.635381) (xy 187.513395 73.003485) (xy 187.993179 72.396467)
   (xy 188.416912 71.825806) (xy 188.775788 71.30298) (xy 188.928153 71.063092) (xy 189.061001 70.839466) (xy 189.173232 70.633538)
   (xy 189.263745 70.446743) (xy 189.567927 69.824561) (xy 189.910614 69.226171) (xy 190.29011 68.652048) (xy 190.704722 68.102671)
   (xy 191.152754 67.578514) (xy 191.632512 67.080056) (xy 192.142299 66.607772) (xy 192.680423 66.16214) (xy 193.245187 65.743637)
   (xy 193.834896 65.352738) (xy 194.447857 64.98992) (xy 195.082373 64.655661) (xy 195.73675 64.350437) (xy 196.409294 64.074725)
   (xy 197.098308 63.829001) (xy 197.802099 63.613743) (xy 198.518972 63.429426) (xy 199.24723 63.276528) (xy 199.985181 63.155525)
   (xy 200.731128 63.066894) (xy 201.483377 63.011112) (xy 202.240232 62.988655))
  (stroke (width 0.1) (type solid)) (fill no) (layer "Edge.Cuts"))
 (segment (start 203.015 101.5) (end 202 101.5) (width 0.2) (layer "F.Cu") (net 7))
 (segment (start 210.188821 110.701) (end 217.811179 110.701) (width 0.2) (layer "F.Cu") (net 7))
 (segment (start 224.985 103.527179) (end 224.985 101.5) (width 0.2) (layer "F.Cu") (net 7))
 (segment (start 202 101.5) (end 198.5 98) (width 0.2) (layer "F.Cu") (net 7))
 (segment (start 203.015 101.5) (end 203.015 103.527179) (width 0.2) (layer "F.Cu") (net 7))
 (segment (start 217.811179 110.701) (end 224.985 103.527179) (width 0.2) (layer "F.Cu") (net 7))
 (segment (start 198.5 98) (end 192 98) (width 0.2) (layer "F.Cu") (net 7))
 (segment (start 203.015 103.527179) (end 210.188821 110.701) (width 0.2) (layer "F.Cu") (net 7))
 (segment (start 209.5 74.265) (end 208.765 74.265) (width 0.2) (layer "F.Cu") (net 4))
 (segment (start 209.5 97) (end 214 101.5) (width 0.2) (layer "F.Cu") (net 4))
 (segment (start 208.765 74.265) (end 208.53 74.5) (width 0.2) (layer "F.Cu") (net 4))
 (segment (start 208.53 74.5) (end 193.5 74.5) (width 0.2) (layer "F.Cu") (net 4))
 (segment (start 209.5 74.265) (end 209.5 97) (width 0.2) (layer "F.Cu") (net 4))
 (segment (start 216.5 82) (end 216.5 78.725) (width 0.2) (layer "F.Cu") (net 5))
 (segment (start 216.5 78.725) (end 209.5 71.725) (width 0.2) (layer "F.Cu") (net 5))
 (segment (start 195.96 79.5) (end 190.96 74.5) (width 0.2) (layer "F.Cu") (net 1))
 (segment (start 195.96 85.56) (end 195.96 79.5) (width 0.2) (layer "F.Cu") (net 1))
 (segment (start 213.96 84.54) (end 213.96 77.09724) (width 0.2) (layer "F.Cu") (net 2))
 (segment (start 198.5 93.5) (end 198.5 88.1) (width 0.2) (layer "F.Cu") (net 2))
 (segment (start 213.96 77.09724) (end 209.97676 73.114) (width 0.2) (layer "F.Cu") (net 2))
 (segment (start 189.759 80.802913) (end 197.056087 88.1) (width 0.2) (layer "F.Cu") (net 2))
 (segment (start 190.647529 73.114) (end 189.759 74.002529) (width 0.2) (layer "F.Cu") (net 2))
 (segment (start 197.056087 88.1) (end 198.5 88.1) (width 0.2) (layer "F.Cu") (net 2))
 (segment (start 189.759 74.002529) (end 189.759 80.802913) (width 0.2) (layer "F.Cu") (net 2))
 (segment (start 198.5 93.5) (end 192 93.5) (width 0.2) (layer "F.Cu") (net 2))
 (segment (start 209.97676 73.114) (end 190.647529 73.114) (width 0.2) (layer "F.Cu") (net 2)))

